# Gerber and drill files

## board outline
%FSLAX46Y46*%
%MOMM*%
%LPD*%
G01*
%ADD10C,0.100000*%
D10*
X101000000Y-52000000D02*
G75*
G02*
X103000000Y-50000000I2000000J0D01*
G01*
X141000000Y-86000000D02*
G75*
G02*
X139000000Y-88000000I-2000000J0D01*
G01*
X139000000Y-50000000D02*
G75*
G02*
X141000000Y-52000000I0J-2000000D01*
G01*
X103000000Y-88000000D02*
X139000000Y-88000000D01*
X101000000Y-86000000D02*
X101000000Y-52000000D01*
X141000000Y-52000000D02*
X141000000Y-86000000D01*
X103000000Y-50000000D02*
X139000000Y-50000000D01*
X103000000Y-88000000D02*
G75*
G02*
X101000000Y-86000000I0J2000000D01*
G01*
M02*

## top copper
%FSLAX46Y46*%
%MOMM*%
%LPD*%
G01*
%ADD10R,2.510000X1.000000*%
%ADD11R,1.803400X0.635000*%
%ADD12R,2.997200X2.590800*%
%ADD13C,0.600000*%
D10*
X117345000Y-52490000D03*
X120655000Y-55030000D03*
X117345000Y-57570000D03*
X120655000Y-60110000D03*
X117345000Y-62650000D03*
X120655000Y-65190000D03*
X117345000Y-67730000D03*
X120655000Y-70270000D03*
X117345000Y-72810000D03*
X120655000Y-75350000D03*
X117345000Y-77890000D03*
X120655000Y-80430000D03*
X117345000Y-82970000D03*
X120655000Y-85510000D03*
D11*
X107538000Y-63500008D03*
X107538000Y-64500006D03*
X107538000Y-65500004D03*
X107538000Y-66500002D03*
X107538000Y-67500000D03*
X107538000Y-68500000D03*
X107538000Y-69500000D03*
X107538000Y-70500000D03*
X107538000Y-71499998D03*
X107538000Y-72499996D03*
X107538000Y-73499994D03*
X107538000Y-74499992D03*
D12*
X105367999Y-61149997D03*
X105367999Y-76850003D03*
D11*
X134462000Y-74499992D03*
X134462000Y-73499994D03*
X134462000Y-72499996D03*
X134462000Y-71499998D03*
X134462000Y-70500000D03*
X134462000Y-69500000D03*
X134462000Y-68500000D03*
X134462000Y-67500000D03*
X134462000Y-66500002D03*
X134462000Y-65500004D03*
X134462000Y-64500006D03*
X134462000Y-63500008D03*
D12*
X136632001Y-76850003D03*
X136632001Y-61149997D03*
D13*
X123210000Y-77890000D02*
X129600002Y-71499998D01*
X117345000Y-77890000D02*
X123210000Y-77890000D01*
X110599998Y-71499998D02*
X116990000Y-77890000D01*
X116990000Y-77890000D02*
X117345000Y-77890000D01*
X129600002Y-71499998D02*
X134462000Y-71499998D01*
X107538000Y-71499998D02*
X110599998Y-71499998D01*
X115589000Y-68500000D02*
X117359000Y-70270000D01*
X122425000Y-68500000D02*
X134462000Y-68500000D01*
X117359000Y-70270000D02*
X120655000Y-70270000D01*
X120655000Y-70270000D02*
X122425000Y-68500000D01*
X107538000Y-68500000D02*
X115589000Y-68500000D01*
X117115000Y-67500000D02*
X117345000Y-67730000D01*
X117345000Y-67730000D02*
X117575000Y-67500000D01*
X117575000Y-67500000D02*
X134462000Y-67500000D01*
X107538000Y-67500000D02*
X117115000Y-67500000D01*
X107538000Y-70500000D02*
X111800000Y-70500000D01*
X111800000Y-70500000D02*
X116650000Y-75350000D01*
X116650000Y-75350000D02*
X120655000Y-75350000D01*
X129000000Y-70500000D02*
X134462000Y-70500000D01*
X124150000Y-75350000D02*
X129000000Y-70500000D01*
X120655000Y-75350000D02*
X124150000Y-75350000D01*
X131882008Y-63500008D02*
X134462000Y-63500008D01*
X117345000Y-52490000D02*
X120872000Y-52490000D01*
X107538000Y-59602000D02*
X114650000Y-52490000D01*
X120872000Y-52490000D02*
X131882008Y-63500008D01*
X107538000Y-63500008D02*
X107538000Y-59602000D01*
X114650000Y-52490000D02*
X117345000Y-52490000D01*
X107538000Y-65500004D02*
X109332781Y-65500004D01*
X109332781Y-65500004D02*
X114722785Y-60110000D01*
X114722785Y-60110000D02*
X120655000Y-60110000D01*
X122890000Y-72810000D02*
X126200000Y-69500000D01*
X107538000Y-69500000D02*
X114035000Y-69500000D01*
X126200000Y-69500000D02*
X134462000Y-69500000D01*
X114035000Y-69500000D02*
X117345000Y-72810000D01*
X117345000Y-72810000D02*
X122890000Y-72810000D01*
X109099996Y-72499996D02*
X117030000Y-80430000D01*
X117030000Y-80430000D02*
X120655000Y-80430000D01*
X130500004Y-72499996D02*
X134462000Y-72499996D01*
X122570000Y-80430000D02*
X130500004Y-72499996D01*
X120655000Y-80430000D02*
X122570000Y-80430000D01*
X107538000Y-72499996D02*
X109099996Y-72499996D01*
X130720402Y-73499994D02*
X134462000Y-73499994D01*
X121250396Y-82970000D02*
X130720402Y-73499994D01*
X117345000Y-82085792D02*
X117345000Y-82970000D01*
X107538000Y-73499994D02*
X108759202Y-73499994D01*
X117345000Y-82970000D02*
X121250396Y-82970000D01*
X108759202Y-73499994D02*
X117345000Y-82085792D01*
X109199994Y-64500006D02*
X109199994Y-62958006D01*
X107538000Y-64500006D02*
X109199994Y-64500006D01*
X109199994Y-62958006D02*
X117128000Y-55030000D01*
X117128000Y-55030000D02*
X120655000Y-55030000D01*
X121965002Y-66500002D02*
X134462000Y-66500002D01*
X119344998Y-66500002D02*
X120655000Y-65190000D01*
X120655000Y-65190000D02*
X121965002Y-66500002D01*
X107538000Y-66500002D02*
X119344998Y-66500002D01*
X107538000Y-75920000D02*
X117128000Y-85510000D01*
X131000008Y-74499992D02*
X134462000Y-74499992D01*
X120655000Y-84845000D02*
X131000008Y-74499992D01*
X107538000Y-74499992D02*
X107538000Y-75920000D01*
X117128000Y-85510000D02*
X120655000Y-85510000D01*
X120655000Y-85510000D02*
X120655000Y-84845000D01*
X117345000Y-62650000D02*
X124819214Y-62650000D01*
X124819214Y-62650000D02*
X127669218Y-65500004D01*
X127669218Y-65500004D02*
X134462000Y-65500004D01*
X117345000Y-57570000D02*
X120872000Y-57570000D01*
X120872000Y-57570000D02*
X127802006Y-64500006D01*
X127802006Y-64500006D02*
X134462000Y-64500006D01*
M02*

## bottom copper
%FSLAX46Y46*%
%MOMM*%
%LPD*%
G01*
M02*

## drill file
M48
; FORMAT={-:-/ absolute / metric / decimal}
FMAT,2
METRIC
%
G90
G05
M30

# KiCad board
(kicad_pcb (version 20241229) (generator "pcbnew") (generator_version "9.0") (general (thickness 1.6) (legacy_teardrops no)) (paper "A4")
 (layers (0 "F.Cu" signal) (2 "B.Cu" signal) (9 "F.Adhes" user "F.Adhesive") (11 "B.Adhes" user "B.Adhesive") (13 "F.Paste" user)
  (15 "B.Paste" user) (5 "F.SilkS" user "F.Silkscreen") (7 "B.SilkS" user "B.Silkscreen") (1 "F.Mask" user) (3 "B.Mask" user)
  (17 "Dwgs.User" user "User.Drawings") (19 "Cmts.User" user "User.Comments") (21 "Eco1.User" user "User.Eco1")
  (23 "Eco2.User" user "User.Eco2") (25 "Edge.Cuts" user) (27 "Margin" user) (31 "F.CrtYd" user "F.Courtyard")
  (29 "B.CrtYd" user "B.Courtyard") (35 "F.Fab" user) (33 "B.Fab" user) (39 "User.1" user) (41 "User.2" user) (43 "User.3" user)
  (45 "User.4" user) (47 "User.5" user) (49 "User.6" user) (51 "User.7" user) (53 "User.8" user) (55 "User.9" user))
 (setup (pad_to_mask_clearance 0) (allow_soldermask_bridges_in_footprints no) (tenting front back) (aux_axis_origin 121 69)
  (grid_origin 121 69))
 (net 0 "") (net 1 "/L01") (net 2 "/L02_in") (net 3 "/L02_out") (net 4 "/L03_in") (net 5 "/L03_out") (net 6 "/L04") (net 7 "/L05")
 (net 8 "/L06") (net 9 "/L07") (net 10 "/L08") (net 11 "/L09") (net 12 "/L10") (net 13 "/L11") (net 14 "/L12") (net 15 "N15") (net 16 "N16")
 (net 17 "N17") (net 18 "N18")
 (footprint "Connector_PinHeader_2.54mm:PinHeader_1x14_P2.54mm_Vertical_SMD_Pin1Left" (layer "F.Cu") (at 119 69)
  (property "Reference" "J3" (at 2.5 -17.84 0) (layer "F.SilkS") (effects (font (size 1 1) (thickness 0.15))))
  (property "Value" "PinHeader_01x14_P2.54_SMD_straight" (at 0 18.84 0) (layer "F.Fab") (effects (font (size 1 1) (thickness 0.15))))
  (pad "1" smd rect (at -1.655 -16.51) (size 2.51 1) (layers "F.Cu" "F.Mask" "F.Paste") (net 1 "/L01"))
  (pad "2" smd rect (at 1.655 -13.97) (size 2.51 1) (layers "F.Cu" "F.Mask" "F.Paste") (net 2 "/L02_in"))
  (pad "3" smd rect (at -1.655 -11.43) (size 2.51 1) (layers "F.Cu" "F.Mask" "F.Paste") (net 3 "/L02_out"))
  (pad "4" smd rect (at 1.655 -8.89) (size 2.51 1) (layers "F.Cu" "F.Mask" "F.Paste") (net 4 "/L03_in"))
  (pad "5" smd rect (at -1.655 -6.35) (size 2.51 1) (layers "F.Cu" "F.Mask" "F.Paste") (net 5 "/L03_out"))
  (pad "6" smd rect (at 1.655 -3.81) (size 2.51 1) (layers "F.Cu" "F.Mask" "F.Paste") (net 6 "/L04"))
  (pad "7" smd rect (at -1.655 -1.27) (size 2.51 1) (layers "F.Cu" "F.Mask" "F.Paste") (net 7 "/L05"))
  (pad "8" smd rect (at 1.655 1.27) (size 2.51 1) (layers "F.Cu" "F.Mask" "F.Paste") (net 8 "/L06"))
  (pad "9" smd rect (at -1.655 3.81) (size 2.51 1) (layers "F.Cu" "F.Mask" "F.Paste") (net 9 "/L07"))
  (pad "10" smd rect (at 1.655 6.35) (size 2.51 1) (layers "F.Cu" "F.Mask" "F.Paste") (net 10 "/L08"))
  (pad "11" smd rect (at -1.655 8.89) (size 2.51 1) (layers "F.Cu" "F.Mask" "F.Paste") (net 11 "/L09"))
  (pad "12" smd rect (at 1.655 11.43) (size 2.51 1) (layers "F.Cu" "F.Mask" "F.Paste") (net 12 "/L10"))
  (pad "13" smd rect (at -1.655 13.97) (size 2.51 1) (layers "F.Cu" "F.Mask" "F.Paste") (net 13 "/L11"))
  (pad "14" smd rect (at 1.655 16.51) (size 2.51 1) (layers "F.Cu" "F.Mask" "F.Paste") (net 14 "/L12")))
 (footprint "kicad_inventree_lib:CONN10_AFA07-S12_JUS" (layer "F.Cu") (at 103.982 69 -90)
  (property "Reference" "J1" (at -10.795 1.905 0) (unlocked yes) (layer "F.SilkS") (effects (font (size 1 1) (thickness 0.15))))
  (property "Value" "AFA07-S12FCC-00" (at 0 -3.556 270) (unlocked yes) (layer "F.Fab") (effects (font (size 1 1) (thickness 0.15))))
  (pad "1" smd rect (at -5.499992 -3.556 270) (size 0.635 1.8034) (layers "F.Cu" "F.Mask" "F.Paste") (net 1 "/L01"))
  (pad "2" smd rect (at -4.499994 -3.556 270) (size 0.635 1.8034) (layers "F.Cu" "F.Mask" "F.Paste") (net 2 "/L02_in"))
  (pad "3" smd rect (at -3.499996 -3.556 270) (size 0.635 1.8034) (layers "F.Cu" "F.Mask" "F.Paste") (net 4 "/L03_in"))
  (pad "4" smd rect (at -2.499998 -3.556 270) (size 0.635 1.8034) (layers "F.Cu" "F.Mask" "F.Paste") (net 6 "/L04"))
  (pad "5" smd rect (at -1.5 -3.556 270) (size 0.635 1.8034) (layers "F.Cu" "F.Mask" "F.Paste") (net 7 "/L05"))
  (pad "6" smd rect (at -0.5 -3.556 270) (size 0.635 1.8034) (layers "F.Cu" "F.Mask" "F.Paste") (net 8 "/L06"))
  (pad "7" smd rect (at 0.5 -3.556 270) (size 0.635 1.8034) (layers "F.Cu" "F.Mask" "F.Paste") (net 9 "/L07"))
  (pad "8" smd rect (at 1.5 -3.556 270) (size 0.635 1.8034) (layers "F.Cu" "F.Mask" "F.Paste") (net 10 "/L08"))
  (pad "9" smd rect (at 2.499998 -3.556 270) (size 0.635 1.8034) (layers "F.Cu" "F.Mask" "F.Paste") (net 11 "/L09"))
  (pad "10" smd rect (at 3.499996 -3.556 270) (size 0.635 1.8034) (layers "F.Cu" "F.Mask" "F.Paste") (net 12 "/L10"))
  (pad "11" smd rect (at 4.499994 -3.556 270) (size 0.635 1.8034) (layers "F.Cu" "F.Mask" "F.Paste") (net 13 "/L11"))
  (pad "12" smd rect (at 5.499992 -3.556 270) (size 0.635 1.8034) (layers "F.Cu" "F.Mask" "F.Paste") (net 14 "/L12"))
  (pad "13" smd rect (at -7.850003 -1.385999 270) (size 2.5908 2.9972) (layers "F.Cu" "F.Mask" "F.Paste") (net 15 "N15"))
  (pad "13" smd rect (at 7.850003 -1.385999 270) (size 2.5908 2.9972) (layers "F.Cu" "F.Mask" "F.Paste") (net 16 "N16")))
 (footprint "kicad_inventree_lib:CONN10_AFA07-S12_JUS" (layer "F.Cu") (at 138.018 69 90)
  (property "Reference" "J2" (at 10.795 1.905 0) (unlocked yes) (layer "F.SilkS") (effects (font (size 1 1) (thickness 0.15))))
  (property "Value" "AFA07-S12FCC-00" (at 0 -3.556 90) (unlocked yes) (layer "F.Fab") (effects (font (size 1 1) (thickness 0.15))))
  (pad "1" smd rect (at -5.499992 -3.556 90) (size 0.635 1.8034) (layers "F.Cu" "F.Mask" "F.Paste") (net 14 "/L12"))
  (pad "2" smd rect (at -4.499994 -3.556 90) (size 0.635 1.8034) (layers "F.Cu" "F.Mask" "F.Paste") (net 13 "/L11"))
  (pad "3" smd rect (at -3.499996 -3.556 90) (size 0.635 1.8034) (layers "F.Cu" "F.Mask" "F.Paste") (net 12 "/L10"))
  (pad "4" smd rect (at -2.499998 -3.556 90) (size 0.635 1.8034) (layers "F.Cu" "F.Mask" "F.Paste") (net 11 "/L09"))
  (pad "5" smd rect (at -1.5 -3.556 90) (size 0.635 1.8034) (layers "F.Cu" "F.Mask" "F.Paste") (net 10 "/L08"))
  (pad "6" smd rect (at -0.5 -3.556 90) (size 0.635 1.8034) (layers "F.Cu" "F.Mask" "F.Paste") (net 9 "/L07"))
  (pad "7" smd rect (at 0.5 -3.556 90) (size 0.635 1.8034) (layers "F.Cu" "F.Mask" "F.Paste") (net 8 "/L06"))
  (pad "8" smd rect (at 1.5 -3.556 90) (size 0.635 1.8034) (layers "F.Cu" "F.Mask" "F.Paste") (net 7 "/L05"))
  (pad "9" smd rect (at 2.499998 -3.556 90) (size 0.635 1.8034) (layers "F.Cu" "F.Mask" "F.Paste") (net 6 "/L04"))
  (pad "10" smd rect (at 3.499996 -3.556 90) (size 0.635 1.8034) (layers "F.Cu" "F.Mask" "F.Paste") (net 5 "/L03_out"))
  (pad "11" smd rect (at 4.499994 -3.556 90) (size 0.635 1.8034) (layers "F.Cu" "F.Mask" "F.Paste") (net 3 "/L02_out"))
  (pad "12" smd rect (at 5.499992 -3.556 90) (size 0.635 1.8034) (layers "F.Cu" "F.Mask" "F.Paste") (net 1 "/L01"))
  (pad "13" smd rect (at -7.850003 -1.385999 90) (size 2.5908 2.9972) (layers "F.Cu" "F.Mask" "F.Paste") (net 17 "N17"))
  (pad "13" smd rect (at 7.850003 -1.385999 90) (size 2.5908 2.9972) (layers "F.Cu" "F.Mask" "F.Paste") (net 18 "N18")))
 (gr_arc (start 101 52) (mid 101.585786 50.585786) (end 103 50) (stroke (width 0.1) (type default)) (layer "Edge.Cuts"))
 (gr_arc (start 141 86) (mid 140.414214 87.414214) (end 139 88) (stroke (width 0.1) (type default)) (layer "Edge.Cuts"))
 (gr_arc (start 139 50) (mid 140.414214 50.585786) (end 141 52) (stroke (width 0.1) (type default)) (layer "Edge.Cuts"))
 (gr_line (start 103 88) (end 139 88) (stroke (width 0.1) (type default)) (layer "Edge.Cuts"))
 (gr_line (start 101 86) (end 101 52) (stroke (width 0.1) (type default)) (layer "Edge.Cuts"))
 (gr_line (start 141 52) (end 141 86) (stroke (width 0.1) (type default)) (layer "Edge.Cuts"))
 (gr_line (start 103 50) (end 139 50) (stroke (width 0.1) (type default)) (layer "Edge.Cuts"))
 (gr_arc (start 103 88) (mid 101.585786 87.414214) (end 101 86) (stroke (width 0.1) (type default)) (layer "Edge.Cuts"))
 (segment (start 123.21 77.89) (end 129.600002 71.499998) (width 0.6) (layer "F.Cu") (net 11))
 (segment (start 117.345 77.89) (end 123.21 77.89) (width 0.6) (layer "F.Cu") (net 11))
 (segment (start 110.599998 71.499998) (end 116.99 77.89) (width 0.6) (layer "F.Cu") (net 11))
 (segment (start 116.99 77.89) (end 117.345 77.89) (width 0.6) (layer "F.Cu") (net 11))
 (segment (start 129.600002 71.499998) (end 134.462 71.499998) (width 0.6) (layer "F.Cu") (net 11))
 (segment (start 107.538 71.499998) (end 110.599998 71.499998) (width 0.6) (layer "F.Cu") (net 11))
 (segment (start 115.589 68.5) (end 117.359 70.27) (width 0.6) (layer "F.Cu") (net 8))
 (segment (start 122.425 68.5) (end 134.462 68.5) (width 0.6) (layer "F.Cu") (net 8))
 (segment (start 117.359 70.27) (end 120.655 70.27) (width 0.6) (layer "F.Cu") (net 8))
 (segment (start 120.655 70.27) (end 122.425 68.5) (width 0.6) (layer "F.Cu") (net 8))
 (segment (start 107.538 68.5) (end 115.589 68.5) (width 0.6) (layer "F.Cu") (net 8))
 (segment (start 117.115 67.5) (end 117.345 67.73) (width 0.6) (layer "F.Cu") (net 7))
 (segment (start 117.345 67.73) (end 117.575 67.5) (width 0.6) (layer "F.Cu") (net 7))
 (segment (start 117.575 67.5) (end 134.462 67.5) (width 0.6) (layer "F.Cu") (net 7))
 (segment (start 107.538 67.5) (end 117.115 67.5) (width 0.6) (layer "F.Cu") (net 7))
 (segment (start 107.538 70.5) (end 111.8 70.5) (width 0.6) (layer "F.Cu") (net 10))
 (segment (start 111.8 70.5) (end 116.65 75.35) (width 0.6) (layer "F.Cu") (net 10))
 (segment (start 116.65 75.35) (end 120.655 75.35) (width 0.6) (layer "F.Cu") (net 10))
 (segment (start 129 70.5) (end 134.462 70.5) (width 0.6) (layer "F.Cu") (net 10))
 (segment (start 124.15 75.35) (end 129 70.5) (width 0.6) (layer "F.Cu") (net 10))
 (segment (start 120.655 75.35) (end 124.15 75.35) (width 0.6) (layer "F.Cu") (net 10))
 (segment (start 131.882008 63.500008) (end 134.462 63.500008) (width 0.6) (layer "F.Cu") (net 1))
 (segment (start 117.345 52.49) (end 120.872 52.49) (width 0.6) (layer "F.Cu") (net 1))
 (segment (start 107.538 59.602) (end 114.65 52.49) (width 0.6) (layer "F.Cu") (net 1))
 (segment (start 120.872 52.49) (end 131.882008 63.500008) (width 0.6) (layer "F.Cu") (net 1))
 (segment (start 107.538 63.500008) (end 107.538 59.602) (width 0.6) (layer "F.Cu") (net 1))
 (segment (start 114.65 52.49) (end 117.345 52.49) (width 0.6) (layer "F.Cu") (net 1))
 (segment (start 107.538 65.500004) (end 109.332781 65.500004) (width 0.6) (layer "F.Cu") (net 4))
 (segment (start 109.332781 65.500004) (end 114.722785 60.11) (width 0.6) (layer "F.Cu") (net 4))
 (segment (start 114.722785 60.11) (end 120.655 60.11) (width 0.6) (layer "F.Cu") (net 4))
 (segment (start 122.89 72.81) (end 126.2 69.5) (width 0.6) (layer "F.Cu") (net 9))
 (segment (start 107.538 69.5) (end 114.035 69.5) (width 0.6) (layer "F.Cu") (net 9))
 (segment (start 126.2 69.5) (end 134.462 69.5) (width 0.6) (layer "F.Cu") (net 9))
 (segment (start 114.035 69.5) (end 117.345 72.81) (width 0.6) (layer "F.Cu") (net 9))
 (segment (start 117.345 72.81) (end 122.89 72.81) (width 0.6) (layer "F.Cu") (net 9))
 (segment (start 109.099996 72.499996) (end 117.03 80.43) (width 0.6) (layer "F.Cu") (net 12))
 (segment (start 117.03 80.43) (end 120.655 80.43) (width 0.6) (layer "F.Cu") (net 12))
 (segment (start 130.500004 72.499996) (end 134.462 72.499996) (width 0.6) (layer "F.Cu") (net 12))
 (segment (start 122.57 80.43) (end 130.500004 72.499996) (width 0.6) (layer "F.Cu") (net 12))
 (segment (start 120.655 80.43) (end 122.57 80.43) (width 0.6) (layer "F.Cu") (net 12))
 (segment (start 107.538 72.499996) (end 109.099996 72.499996) (width 0.6) (layer "F.Cu") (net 12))
 (segment (start 130.720402 73.499994) (end 134.462 73.499994) (width 0.6) (layer "F.Cu") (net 13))
 (segment (start 121.250396 82.97) (end 130.720402 73.499994) (width 0.6) (layer "F.Cu") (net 13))
 (segment (start 117.345 82.085792) (end 117.345 82.97) (width 0.6) (layer "F.Cu") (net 13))
 (segment (start 107.538 73.499994) (end 108.759202 73.499994) (width 0.6) (layer "F.Cu") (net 13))
 (segment (start 117.345 82.97) (end 121.250396 82.97) (width 0.6) (layer "F.Cu") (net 13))
 (segment (start 108.759202 73.499994) (end 117.345 82.085792) (width 0.6) (layer "F.Cu") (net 13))
 (segment (start 109.199994 64.500006) (end 109.199994 62.958006) (width 0.6) (layer "F.Cu") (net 2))
 (segment (start 107.538 64.500006) (end 109.199994 64.500006) (width 0.6) (layer "F.Cu") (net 2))
 (segment (start 109.199994 62.958006) (end 117.128 55.03) (width 0.6) (layer "F.Cu") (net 2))
 (segment (start 117.128 55.03) (end 120.655 55.03) (width 0.6) (layer "F.Cu") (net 2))
 (segment (start 121.965002 66.500002) (end 134.462 66.500002) (width 0.6) (layer "F.Cu") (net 6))
 (segment (start 119.344998 66.500002) (end 120.655 65.19) (width 0.6) (layer "F.Cu") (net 6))
 (segment (start 120.655 65.19) (end 121.965002 66.500002) (width 0.6) (layer "F.Cu") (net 6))
 (segment (start 107.538 66.500002) (end 119.344998 66.500002) (width 0.6) (layer "F.Cu") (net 6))
 (segment (start 107.538 75.92) (end 117.128 85.51) (width 0.6) (layer "F.Cu") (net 14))
 (segment (start 131.000008 74.499992) (end 134.462 74.499992) (width 0.6) (layer "F.Cu") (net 14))
 (segment (start 120.655 84.845) (end 131.000008 74.499992) (width 0.6) (layer "F.Cu") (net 14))
 (segment (start 107.538 74.499992) (end 107.538 75.92) (width 0.6) (layer "F.Cu") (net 14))
 (segment (start 117.128 85.51) (end 120.655 85.51) (width 0.6) (layer "F.Cu") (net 14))
 (segment (start 120.655 85.51) (end 120.655 84.845) (width 0.6) (layer "F.Cu") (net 14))
 (segment (start 117.345 62.65) (end 124.819214 62.65) (width 0.6) (layer "F.Cu") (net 5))
 (segment (start 124.819214 62.65) (end 127.669218 65.500004) (width 0.6) (layer "F.Cu") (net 5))
 (segment (start 127.669218 65.500004) (end 134.462 65.500004) (width 0.6) (layer "F.Cu") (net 5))
 (segment (start 117.345 57.57) (end 120.872 57.57) (width 0.6) (layer "F.Cu") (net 3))
 (segment (start 120.872 57.57) (end 127.802006 64.500006) (width 0.6) (layer "F.Cu") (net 3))
 (segment (start 127.802006 64.500006) (end 134.462 64.500006) (width 0.6) (layer "F.Cu") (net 3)))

